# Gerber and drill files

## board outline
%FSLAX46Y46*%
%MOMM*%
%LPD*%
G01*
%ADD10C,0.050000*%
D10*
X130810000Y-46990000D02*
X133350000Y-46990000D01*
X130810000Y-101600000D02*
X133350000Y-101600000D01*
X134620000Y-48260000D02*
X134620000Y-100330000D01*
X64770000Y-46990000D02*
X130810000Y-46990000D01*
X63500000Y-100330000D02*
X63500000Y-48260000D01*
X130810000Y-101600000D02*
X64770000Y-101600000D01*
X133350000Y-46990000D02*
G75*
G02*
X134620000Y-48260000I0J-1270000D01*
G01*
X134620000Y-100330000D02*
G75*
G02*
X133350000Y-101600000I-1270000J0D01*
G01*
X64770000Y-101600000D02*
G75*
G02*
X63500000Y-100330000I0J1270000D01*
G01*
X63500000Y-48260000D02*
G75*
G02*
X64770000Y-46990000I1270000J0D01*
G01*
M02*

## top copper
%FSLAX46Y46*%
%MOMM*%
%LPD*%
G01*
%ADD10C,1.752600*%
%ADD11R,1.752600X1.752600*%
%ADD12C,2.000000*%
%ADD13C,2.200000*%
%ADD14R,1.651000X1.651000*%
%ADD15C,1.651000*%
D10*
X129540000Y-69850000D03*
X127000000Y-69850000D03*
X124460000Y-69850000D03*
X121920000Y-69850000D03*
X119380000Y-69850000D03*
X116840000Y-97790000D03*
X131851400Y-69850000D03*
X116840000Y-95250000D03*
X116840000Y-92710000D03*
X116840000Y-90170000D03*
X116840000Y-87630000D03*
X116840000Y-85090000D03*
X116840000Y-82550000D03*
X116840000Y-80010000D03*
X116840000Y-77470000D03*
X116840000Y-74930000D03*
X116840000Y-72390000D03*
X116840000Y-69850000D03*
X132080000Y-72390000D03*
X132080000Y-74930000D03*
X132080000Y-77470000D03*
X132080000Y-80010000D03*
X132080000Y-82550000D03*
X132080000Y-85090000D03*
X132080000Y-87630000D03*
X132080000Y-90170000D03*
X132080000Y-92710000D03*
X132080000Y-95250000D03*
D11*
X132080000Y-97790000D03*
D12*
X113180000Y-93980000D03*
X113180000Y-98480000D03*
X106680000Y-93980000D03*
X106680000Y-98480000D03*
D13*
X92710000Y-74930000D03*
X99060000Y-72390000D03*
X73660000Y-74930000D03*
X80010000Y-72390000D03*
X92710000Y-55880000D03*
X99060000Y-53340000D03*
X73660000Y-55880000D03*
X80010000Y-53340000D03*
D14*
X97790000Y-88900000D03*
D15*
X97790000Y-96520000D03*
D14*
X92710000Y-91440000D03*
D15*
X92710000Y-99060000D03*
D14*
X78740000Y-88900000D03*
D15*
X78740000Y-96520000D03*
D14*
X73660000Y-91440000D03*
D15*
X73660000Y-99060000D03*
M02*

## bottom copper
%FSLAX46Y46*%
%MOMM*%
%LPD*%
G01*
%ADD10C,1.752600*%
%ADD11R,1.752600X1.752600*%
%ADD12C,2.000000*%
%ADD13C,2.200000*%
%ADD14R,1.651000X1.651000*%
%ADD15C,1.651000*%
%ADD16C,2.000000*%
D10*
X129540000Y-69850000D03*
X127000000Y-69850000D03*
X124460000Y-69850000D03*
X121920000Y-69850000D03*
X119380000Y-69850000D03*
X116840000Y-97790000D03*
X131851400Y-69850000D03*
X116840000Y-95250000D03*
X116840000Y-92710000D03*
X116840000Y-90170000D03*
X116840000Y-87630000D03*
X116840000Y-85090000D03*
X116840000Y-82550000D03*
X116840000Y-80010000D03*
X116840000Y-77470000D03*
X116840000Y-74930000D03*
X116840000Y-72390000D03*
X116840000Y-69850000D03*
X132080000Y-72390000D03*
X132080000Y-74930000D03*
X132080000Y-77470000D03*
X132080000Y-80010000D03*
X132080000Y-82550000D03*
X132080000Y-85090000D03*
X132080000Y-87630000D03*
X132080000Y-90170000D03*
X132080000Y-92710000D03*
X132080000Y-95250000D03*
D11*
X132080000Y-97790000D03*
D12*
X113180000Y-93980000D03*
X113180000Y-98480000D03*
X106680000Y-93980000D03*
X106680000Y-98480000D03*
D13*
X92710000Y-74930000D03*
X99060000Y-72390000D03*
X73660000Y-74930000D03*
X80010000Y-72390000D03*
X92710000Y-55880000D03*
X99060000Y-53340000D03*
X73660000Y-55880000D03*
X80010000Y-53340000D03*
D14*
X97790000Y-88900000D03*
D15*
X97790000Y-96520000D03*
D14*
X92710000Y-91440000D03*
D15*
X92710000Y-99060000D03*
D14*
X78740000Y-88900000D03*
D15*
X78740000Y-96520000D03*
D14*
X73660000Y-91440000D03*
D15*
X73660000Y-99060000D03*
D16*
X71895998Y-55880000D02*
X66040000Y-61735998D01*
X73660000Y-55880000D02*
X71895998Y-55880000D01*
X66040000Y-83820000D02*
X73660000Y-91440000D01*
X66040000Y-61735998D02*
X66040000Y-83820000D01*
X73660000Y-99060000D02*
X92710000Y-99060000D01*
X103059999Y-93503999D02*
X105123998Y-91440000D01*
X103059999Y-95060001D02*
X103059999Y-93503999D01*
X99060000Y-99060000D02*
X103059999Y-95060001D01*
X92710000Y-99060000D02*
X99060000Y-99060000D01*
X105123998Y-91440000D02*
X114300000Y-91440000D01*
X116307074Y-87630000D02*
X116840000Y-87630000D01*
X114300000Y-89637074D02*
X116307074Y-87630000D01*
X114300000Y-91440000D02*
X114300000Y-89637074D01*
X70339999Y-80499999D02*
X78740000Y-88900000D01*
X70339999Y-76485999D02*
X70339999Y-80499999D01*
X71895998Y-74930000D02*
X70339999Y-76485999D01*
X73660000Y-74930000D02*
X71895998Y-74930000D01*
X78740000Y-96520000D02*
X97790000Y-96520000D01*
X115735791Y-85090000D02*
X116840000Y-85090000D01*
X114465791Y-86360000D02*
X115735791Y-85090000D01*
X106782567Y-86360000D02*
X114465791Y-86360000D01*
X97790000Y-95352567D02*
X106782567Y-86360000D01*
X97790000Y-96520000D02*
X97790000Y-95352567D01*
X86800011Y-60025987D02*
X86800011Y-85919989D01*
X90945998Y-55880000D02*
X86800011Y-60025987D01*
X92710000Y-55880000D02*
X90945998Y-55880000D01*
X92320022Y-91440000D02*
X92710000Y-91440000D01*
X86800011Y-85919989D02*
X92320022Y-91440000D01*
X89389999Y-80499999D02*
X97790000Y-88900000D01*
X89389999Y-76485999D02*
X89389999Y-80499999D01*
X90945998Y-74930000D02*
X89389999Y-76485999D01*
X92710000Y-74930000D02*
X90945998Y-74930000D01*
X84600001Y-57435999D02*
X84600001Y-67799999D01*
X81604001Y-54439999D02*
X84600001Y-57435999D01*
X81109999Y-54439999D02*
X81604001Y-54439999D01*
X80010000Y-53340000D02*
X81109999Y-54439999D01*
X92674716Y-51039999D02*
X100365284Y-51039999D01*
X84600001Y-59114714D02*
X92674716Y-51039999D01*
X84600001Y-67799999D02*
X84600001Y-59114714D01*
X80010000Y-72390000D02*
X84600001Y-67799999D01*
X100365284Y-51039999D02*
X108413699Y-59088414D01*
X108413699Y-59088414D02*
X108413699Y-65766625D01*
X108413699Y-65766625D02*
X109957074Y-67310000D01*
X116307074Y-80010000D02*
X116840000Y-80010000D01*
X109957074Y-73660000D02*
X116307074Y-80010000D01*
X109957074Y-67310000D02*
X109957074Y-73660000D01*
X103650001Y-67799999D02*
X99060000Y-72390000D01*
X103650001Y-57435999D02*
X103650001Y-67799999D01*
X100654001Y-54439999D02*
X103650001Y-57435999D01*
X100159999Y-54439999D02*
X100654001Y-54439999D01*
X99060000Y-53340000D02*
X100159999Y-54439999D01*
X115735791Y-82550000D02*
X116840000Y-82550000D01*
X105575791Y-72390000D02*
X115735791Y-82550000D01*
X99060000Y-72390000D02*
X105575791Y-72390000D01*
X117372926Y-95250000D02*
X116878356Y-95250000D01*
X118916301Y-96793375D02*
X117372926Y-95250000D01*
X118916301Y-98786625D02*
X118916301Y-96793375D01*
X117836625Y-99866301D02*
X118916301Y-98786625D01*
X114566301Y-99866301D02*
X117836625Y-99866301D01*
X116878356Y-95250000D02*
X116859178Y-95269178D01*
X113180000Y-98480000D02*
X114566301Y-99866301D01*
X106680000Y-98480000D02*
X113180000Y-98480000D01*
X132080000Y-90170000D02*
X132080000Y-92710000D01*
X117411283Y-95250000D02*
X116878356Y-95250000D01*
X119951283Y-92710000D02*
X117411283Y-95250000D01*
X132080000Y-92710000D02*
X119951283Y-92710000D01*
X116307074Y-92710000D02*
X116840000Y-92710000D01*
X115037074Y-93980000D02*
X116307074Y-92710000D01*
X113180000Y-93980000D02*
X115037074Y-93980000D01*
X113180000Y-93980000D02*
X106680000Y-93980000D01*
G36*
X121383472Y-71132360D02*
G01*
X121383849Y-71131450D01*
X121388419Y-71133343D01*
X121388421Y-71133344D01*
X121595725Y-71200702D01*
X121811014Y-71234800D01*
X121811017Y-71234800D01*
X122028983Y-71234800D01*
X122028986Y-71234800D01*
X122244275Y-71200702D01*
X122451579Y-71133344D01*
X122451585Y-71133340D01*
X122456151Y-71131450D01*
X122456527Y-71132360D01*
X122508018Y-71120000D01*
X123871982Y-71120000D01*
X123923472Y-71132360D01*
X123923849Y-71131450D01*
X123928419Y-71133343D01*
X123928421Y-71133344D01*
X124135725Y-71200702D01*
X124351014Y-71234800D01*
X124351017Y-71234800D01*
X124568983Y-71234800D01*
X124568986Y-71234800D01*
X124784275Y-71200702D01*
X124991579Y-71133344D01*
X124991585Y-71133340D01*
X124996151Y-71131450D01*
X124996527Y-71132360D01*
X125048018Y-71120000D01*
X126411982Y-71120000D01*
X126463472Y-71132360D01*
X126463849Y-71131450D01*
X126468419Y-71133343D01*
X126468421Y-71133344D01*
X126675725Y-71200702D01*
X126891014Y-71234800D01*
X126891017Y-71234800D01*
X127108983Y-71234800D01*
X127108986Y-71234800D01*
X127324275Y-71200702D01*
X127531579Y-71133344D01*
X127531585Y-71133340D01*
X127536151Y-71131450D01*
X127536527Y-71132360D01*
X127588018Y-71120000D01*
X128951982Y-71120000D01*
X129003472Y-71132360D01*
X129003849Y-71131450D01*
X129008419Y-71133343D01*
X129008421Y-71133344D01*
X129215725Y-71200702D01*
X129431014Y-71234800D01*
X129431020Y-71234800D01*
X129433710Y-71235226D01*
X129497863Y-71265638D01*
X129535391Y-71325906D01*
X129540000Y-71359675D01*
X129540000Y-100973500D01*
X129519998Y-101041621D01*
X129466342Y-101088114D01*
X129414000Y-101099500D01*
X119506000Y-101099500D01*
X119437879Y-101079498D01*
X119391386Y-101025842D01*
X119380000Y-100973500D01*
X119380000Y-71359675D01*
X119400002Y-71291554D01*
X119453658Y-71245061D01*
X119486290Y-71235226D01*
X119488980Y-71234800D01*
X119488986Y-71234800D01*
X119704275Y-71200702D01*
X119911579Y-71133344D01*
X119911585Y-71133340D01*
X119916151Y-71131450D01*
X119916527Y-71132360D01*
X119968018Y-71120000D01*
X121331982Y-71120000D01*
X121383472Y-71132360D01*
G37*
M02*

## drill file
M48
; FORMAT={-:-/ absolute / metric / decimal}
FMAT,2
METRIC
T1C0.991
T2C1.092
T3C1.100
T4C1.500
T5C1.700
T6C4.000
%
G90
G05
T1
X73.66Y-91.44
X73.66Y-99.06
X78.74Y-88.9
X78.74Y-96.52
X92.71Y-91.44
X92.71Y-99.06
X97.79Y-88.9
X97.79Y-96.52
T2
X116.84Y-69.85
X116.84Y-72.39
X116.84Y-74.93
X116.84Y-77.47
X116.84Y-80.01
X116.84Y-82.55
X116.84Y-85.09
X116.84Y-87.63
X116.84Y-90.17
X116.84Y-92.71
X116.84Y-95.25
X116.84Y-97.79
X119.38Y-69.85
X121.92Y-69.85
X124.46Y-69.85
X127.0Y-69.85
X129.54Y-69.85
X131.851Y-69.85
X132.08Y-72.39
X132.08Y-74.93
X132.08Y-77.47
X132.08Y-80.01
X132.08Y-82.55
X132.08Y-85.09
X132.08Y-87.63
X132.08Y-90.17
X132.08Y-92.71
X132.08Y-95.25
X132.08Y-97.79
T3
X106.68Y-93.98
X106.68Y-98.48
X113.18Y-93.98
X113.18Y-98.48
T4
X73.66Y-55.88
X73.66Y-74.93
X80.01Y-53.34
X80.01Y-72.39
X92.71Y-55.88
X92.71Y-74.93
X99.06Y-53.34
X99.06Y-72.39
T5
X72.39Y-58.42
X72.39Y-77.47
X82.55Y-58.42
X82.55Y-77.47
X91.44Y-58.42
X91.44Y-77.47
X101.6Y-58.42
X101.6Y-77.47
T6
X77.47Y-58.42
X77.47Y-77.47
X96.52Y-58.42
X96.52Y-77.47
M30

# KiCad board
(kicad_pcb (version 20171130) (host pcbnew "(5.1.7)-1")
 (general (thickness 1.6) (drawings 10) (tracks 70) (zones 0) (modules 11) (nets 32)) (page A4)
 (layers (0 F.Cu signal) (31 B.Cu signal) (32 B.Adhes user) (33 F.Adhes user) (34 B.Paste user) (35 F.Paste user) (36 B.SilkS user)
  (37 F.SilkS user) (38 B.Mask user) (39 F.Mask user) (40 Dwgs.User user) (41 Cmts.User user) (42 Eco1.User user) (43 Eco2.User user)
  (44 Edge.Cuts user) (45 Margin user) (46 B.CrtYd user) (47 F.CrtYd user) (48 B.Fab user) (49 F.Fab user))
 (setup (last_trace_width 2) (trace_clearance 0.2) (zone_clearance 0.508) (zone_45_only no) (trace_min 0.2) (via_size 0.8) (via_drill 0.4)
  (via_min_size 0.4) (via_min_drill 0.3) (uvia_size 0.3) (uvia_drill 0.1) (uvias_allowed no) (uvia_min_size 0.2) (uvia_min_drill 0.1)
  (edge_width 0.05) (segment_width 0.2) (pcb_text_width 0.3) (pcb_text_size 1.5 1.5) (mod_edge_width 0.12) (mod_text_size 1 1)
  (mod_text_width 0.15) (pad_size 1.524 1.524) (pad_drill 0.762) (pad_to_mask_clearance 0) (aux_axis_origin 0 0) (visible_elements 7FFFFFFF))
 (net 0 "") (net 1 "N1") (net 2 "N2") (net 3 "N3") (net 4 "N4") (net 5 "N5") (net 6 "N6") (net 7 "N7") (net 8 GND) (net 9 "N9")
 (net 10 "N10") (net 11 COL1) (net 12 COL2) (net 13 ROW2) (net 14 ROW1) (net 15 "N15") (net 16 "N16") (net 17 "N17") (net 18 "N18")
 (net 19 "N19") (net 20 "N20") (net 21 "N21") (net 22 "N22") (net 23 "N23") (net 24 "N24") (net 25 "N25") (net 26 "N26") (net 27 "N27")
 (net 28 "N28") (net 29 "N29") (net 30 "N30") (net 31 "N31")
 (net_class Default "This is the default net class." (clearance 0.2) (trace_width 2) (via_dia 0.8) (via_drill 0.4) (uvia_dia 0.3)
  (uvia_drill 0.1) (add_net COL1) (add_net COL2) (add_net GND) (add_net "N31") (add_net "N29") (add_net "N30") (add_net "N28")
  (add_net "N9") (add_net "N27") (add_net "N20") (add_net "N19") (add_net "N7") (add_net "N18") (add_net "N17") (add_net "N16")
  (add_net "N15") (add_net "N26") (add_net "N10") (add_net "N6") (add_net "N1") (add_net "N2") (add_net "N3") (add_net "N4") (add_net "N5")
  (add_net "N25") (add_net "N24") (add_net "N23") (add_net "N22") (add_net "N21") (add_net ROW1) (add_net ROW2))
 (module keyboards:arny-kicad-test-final (layer F.Cu) (at 124.46 57.15)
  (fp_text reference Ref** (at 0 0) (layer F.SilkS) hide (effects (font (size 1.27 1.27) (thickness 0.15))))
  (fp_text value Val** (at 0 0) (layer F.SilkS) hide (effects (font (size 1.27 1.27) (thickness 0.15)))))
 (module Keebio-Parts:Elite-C (layer F.Cu) (at 124.46 83.82 90)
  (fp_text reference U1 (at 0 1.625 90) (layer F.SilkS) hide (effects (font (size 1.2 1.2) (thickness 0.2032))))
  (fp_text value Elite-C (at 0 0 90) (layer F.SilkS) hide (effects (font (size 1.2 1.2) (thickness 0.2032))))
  (pad 25 thru_hole circle (at 13.97 5.08 90) (size 1.7526 1.7526) (drill 1.0922) (layers *.Cu *.SilkS *.Mask) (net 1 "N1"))
  (pad 26 thru_hole circle (at 13.97 2.54 90) (size 1.7526 1.7526) (drill 1.0922) (layers *.Cu *.SilkS *.Mask) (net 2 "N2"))
  (pad 27 thru_hole circle (at 13.97 0 90) (size 1.7526 1.7526) (drill 1.0922) (layers *.Cu *.SilkS *.Mask) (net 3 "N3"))
  (pad 28 thru_hole circle (at 13.97 -2.54 90) (size 1.7526 1.7526) (drill 1.0922) (layers *.Cu *.SilkS *.Mask) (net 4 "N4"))
  (pad 29 thru_hole circle (at 13.97 -5.08 90) (size 1.7526 1.7526) (drill 1.0922) (layers *.Cu *.SilkS *.Mask) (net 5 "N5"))
  (pad 24 thru_hole circle (at -13.97 -7.62 90) (size 1.7526 1.7526) (drill 1.0922) (layers *.Cu *.SilkS *.Mask) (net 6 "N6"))
  (pad 12 thru_hole circle (at 13.97 7.3914 90) (size 1.7526 1.7526) (drill 1.0922) (layers *.Cu *.SilkS *.Mask) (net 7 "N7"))
  (pad 23 thru_hole circle (at -11.43 -7.62 90) (size 1.7526 1.7526) (drill 1.0922) (layers *.Cu *.SilkS *.Mask) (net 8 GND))
  (pad 22 thru_hole circle (at -8.89 -7.62 90) (size 1.7526 1.7526) (drill 1.0922) (layers *.Cu *.SilkS *.Mask) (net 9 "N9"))
  (pad 21 thru_hole circle (at -6.35 -7.62 90) (size 1.7526 1.7526) (drill 1.0922) (layers *.Cu *.SilkS *.Mask) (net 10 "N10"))
  (pad 20 thru_hole circle (at -3.81 -7.62 90) (size 1.7526 1.7526) (drill 1.0922) (layers *.Cu *.SilkS *.Mask) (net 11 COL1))
  (pad 19 thru_hole circle (at -1.27 -7.62 90) (size 1.7526 1.7526) (drill 1.0922) (layers *.Cu *.SilkS *.Mask) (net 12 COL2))
  (pad 18 thru_hole circle (at 1.27 -7.62 90) (size 1.7526 1.7526) (drill 1.0922) (layers *.Cu *.SilkS *.Mask) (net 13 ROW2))
  (pad 17 thru_hole circle (at 3.81 -7.62 90) (size 1.7526 1.7526) (drill 1.0922) (layers *.Cu *.SilkS *.Mask) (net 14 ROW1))
  (pad 16 thru_hole circle (at 6.35 -7.62 90) (size 1.7526 1.7526) (drill 1.0922) (layers *.Cu *.SilkS *.Mask) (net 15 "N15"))
  (pad 15 thru_hole circle (at 8.89 -7.62 90) (size 1.7526 1.7526) (drill 1.0922) (layers *.Cu *.SilkS *.Mask) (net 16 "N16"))
  (pad 14 thru_hole circle (at 11.43 -7.62 90) (size 1.7526 1.7526) (drill 1.0922) (layers *.Cu *.SilkS *.Mask) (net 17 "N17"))
  (pad 13 thru_hole circle (at 13.97 -7.62 90) (size 1.7526 1.7526) (drill 1.0922) (layers *.Cu *.SilkS *.Mask) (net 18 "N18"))
  (pad 11 thru_hole circle (at 11.43 7.62 90) (size 1.7526 1.7526) (drill 1.0922) (layers *.Cu *.SilkS *.Mask) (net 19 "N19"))
  (pad 10 thru_hole circle (at 8.89 7.62 90) (size 1.7526 1.7526) (drill 1.0922) (layers *.Cu *.SilkS *.Mask) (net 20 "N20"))
  (pad 9 thru_hole circle (at 6.35 7.62 90) (size 1.7526 1.7526) (drill 1.0922) (layers *.Cu *.SilkS *.Mask) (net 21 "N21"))
  (pad 8 thru_hole circle (at 3.81 7.62 90) (size 1.7526 1.7526) (drill 1.0922) (layers *.Cu *.SilkS *.Mask) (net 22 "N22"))
  (pad 7 thru_hole circle (at 1.27 7.62 90) (size 1.7526 1.7526) (drill 1.0922) (layers *.Cu *.SilkS *.Mask) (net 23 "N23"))
  (pad 6 thru_hole circle (at -1.27 7.62 90) (size 1.7526 1.7526) (drill 1.0922) (layers *.Cu *.SilkS *.Mask) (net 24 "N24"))
  (pad 5 thru_hole circle (at -3.81 7.62 90) (size 1.7526 1.7526) (drill 1.0922) (layers *.Cu *.SilkS *.Mask) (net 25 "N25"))
  (pad 4 thru_hole circle (at -6.35 7.62 90) (size 1.7526 1.7526) (drill 1.0922) (layers *.Cu *.SilkS *.Mask) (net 8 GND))
  (pad 3 thru_hole circle (at -8.89 7.62 90) (size 1.7526 1.7526) (drill 1.0922) (layers *.Cu *.SilkS *.Mask) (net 8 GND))
  (pad 2 thru_hole circle (at -11.43 7.62 90) (size 1.7526 1.7526) (drill 1.0922) (layers *.Cu *.SilkS *.Mask) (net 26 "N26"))
  (pad 1 thru_hole rect (at -13.97 7.62 90) (size 1.7526 1.7526) (drill 1.0922) (layers *.Cu *.SilkS *.Mask) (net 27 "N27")))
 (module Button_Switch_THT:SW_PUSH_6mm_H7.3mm (layer F.Cu) (at 106.68 93.98)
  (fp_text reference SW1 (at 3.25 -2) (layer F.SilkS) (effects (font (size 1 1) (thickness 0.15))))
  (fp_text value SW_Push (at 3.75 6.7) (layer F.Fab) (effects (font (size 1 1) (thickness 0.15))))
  (pad 1 thru_hole circle (at 6.5 0 90) (size 2 2) (drill 1.1) (layers *.Cu *.Mask) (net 9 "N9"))
  (pad 2 thru_hole circle (at 6.5 4.5 90) (size 2 2) (drill 1.1) (layers *.Cu *.Mask) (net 8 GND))
  (pad 1 thru_hole circle (at 0 0 90) (size 2 2) (drill 1.1) (layers *.Cu *.Mask) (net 9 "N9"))
  (pad 2 thru_hole circle (at 0 4.5 90) (size 2 2) (drill 1.1) (layers *.Cu *.Mask) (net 8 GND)))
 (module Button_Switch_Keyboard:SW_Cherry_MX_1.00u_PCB (layer F.Cu) (at 99.06 72.39)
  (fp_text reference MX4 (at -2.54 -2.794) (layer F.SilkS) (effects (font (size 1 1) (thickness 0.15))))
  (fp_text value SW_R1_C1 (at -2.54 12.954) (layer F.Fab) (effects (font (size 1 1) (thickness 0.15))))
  (pad "" np_thru_hole circle (at 2.54 5.08) (size 1.7 1.7) (drill 1.7) (layers *.Cu *.Mask))
  (pad "" np_thru_hole circle (at -7.62 5.08) (size 1.7 1.7) (drill 1.7) (layers *.Cu *.Mask))
  (pad "" np_thru_hole circle (at -2.54 5.08) (size 4 4) (drill 4) (layers *.Cu *.Mask))
  (pad 2 thru_hole circle (at -6.35 2.54) (size 2.2 2.2) (drill 1.5) (layers *.Cu *.Mask) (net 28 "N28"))
  (pad 1 thru_hole circle (at 0 0) (size 2.2 2.2) (drill 1.5) (layers *.Cu *.Mask) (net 13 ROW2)))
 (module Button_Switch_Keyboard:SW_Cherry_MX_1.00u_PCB (layer F.Cu) (at 80.01 72.39)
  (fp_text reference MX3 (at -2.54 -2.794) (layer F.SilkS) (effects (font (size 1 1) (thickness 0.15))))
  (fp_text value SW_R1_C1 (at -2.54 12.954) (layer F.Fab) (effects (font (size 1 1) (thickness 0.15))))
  (pad "" np_thru_hole circle (at 2.54 5.08) (size 1.7 1.7) (drill 1.7) (layers *.Cu *.Mask))
  (pad "" np_thru_hole circle (at -7.62 5.08) (size 1.7 1.7) (drill 1.7) (layers *.Cu *.Mask))
  (pad "" np_thru_hole circle (at -2.54 5.08) (size 4 4) (drill 4) (layers *.Cu *.Mask))
  (pad 2 thru_hole circle (at -6.35 2.54) (size 2.2 2.2) (drill 1.5) (layers *.Cu *.Mask) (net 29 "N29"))
  (pad 1 thru_hole circle (at 0 0) (size 2.2 2.2) (drill 1.5) (layers *.Cu *.Mask) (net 14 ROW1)))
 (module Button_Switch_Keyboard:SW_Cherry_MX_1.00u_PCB (layer F.Cu) (at 99.06 53.34)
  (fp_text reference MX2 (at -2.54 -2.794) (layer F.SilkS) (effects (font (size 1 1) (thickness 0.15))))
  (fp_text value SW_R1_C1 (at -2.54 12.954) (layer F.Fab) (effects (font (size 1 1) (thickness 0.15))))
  (pad "" np_thru_hole circle (at 2.54 5.08) (size 1.7 1.7) (drill 1.7) (layers *.Cu *.Mask))
  (pad "" np_thru_hole circle (at -7.62 5.08) (size 1.7 1.7) (drill 1.7) (layers *.Cu *.Mask))
  (pad "" np_thru_hole circle (at -2.54 5.08) (size 4 4) (drill 4) (layers *.Cu *.Mask))
  (pad 2 thru_hole circle (at -6.35 2.54) (size 2.2 2.2) (drill 1.5) (layers *.Cu *.Mask) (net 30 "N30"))
  (pad 1 thru_hole circle (at 0 0) (size 2.2 2.2) (drill 1.5) (layers *.Cu *.Mask) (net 13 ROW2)))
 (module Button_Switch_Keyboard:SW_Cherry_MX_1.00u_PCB (layer F.Cu) (at 80.01 53.34)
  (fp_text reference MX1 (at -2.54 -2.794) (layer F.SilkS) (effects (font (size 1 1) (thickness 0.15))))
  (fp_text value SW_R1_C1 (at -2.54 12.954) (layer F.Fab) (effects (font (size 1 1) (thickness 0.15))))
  (pad "" np_thru_hole circle (at 2.54 5.08) (size 1.7 1.7) (drill 1.7) (layers *.Cu *.Mask))
  (pad "" np_thru_hole circle (at -7.62 5.08) (size 1.7 1.7) (drill 1.7) (layers *.Cu *.Mask))
  (pad "" np_thru_hole circle (at -2.54 5.08) (size 4 4) (drill 4) (layers *.Cu *.Mask))
  (pad 2 thru_hole circle (at -6.35 2.54) (size 2.2 2.2) (drill 1.5) (layers *.Cu *.Mask) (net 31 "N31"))
  (pad 1 thru_hole circle (at 0 0) (size 2.2 2.2) (drill 1.5) (layers *.Cu *.Mask) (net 14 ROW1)))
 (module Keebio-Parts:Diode (layer F.Cu) (at 97.79 92.71 90)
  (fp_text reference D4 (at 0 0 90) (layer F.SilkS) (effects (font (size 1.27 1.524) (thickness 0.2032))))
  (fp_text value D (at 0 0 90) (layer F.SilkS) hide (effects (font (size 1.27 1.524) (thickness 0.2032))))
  (pad 2 thru_hole rect (at 3.81 0 90) (size 1.651 1.651) (drill 0.9906) (layers *.Cu *.SilkS *.Mask) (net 28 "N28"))
  (pad 1 thru_hole circle (at -3.81 0 90) (size 1.651 1.651) (drill 0.9906) (layers *.Cu *.SilkS *.Mask) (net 12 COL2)))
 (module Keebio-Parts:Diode (layer F.Cu) (at 92.71 95.25 90)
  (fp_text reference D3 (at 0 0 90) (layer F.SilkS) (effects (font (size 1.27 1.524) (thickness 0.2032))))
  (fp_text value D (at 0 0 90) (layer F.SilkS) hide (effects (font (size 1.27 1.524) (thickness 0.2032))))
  (pad 2 thru_hole rect (at 3.81 0 90) (size 1.651 1.651) (drill 0.9906) (layers *.Cu *.SilkS *.Mask) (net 30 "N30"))
  (pad 1 thru_hole circle (at -3.81 0 90) (size 1.651 1.651) (drill 0.9906) (layers *.Cu *.SilkS *.Mask) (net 11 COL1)))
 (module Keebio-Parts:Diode (layer F.Cu) (at 78.74 92.71 90)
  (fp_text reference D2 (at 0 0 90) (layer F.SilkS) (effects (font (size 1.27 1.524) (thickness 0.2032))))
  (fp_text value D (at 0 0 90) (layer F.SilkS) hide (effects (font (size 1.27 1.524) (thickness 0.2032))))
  (pad 2 thru_hole rect (at 3.81 0 90) (size 1.651 1.651) (drill 0.9906) (layers *.Cu *.SilkS *.Mask) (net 29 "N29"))
  (pad 1 thru_hole circle (at -3.81 0 90) (size 1.651 1.651) (drill 0.9906) (layers *.Cu *.SilkS *.Mask) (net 12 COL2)))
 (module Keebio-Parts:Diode (layer F.Cu) (at 73.66 95.25 90)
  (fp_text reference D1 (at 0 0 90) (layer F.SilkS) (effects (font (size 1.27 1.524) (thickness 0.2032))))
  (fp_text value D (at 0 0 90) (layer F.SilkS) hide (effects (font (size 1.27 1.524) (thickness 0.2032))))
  (pad 2 thru_hole rect (at 3.81 0 90) (size 1.651 1.651) (drill 0.9906) (layers *.Cu *.SilkS *.Mask) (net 31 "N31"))
  (pad 1 thru_hole circle (at -3.81 0 90) (size 1.651 1.651) (drill 0.9906) (layers *.Cu *.SilkS *.Mask) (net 11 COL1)))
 (gr_line (start 130.81 46.99) (end 133.35 46.99) (layer Edge.Cuts) (width 0.05))
 (gr_line (start 130.81 101.6) (end 133.35 101.6) (layer Edge.Cuts) (width 0.05))
 (gr_line (start 134.62 48.26) (end 134.62 100.33) (layer Edge.Cuts) (width 0.05))
 (gr_line (start 64.77 46.99) (end 130.81 46.99) (layer Edge.Cuts) (width 0.05))
 (gr_line (start 63.5 100.33) (end 63.5 48.26) (layer Edge.Cuts) (width 0.05))
 (gr_line (start 130.81 101.6) (end 64.77 101.6) (layer Edge.Cuts) (width 0.05))
 (gr_arc (start 133.35 48.26) (end 134.62 48.26) (angle -90) (layer Edge.Cuts) (width 0.05))
 (gr_arc (start 133.35 100.33) (end 133.35 101.6) (angle -90) (layer Edge.Cuts) (width 0.05))
 (gr_arc (start 64.77 100.33) (end 63.5 100.33) (angle -90) (layer Edge.Cuts) (width 0.05))
 (gr_arc (start 64.77 48.26) (end 64.77 46.99) (angle -90) (layer Edge.Cuts) (width 0.05))
 (segment (start 71.895998 55.88) (end 66.04 61.735998) (width 2) (layer B.Cu) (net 31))
 (segment (start 73.66 55.88) (end 71.895998 55.88) (width 2) (layer B.Cu) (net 31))
 (segment (start 66.04 83.82) (end 73.66 91.44) (width 2) (layer B.Cu) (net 31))
 (segment (start 66.04 61.735998) (end 66.04 83.82) (width 2) (layer B.Cu) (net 31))
 (segment (start 73.66 99.06) (end 92.71 99.06) (width 2) (layer B.Cu) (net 11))
 (segment (start 103.059999 93.503999) (end 105.123998 91.44) (width 2) (layer B.Cu) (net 11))
 (segment (start 103.059999 95.060001) (end 103.059999 93.503999) (width 2) (layer B.Cu) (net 11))
 (segment (start 99.06 99.06) (end 103.059999 95.060001) (width 2) (layer B.Cu) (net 11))
 (segment (start 92.71 99.06) (end 99.06 99.06) (width 2) (layer B.Cu) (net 11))
 (segment (start 105.123998 91.44) (end 114.3 91.44) (width 2) (layer B.Cu) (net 11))
 (segment (start 116.307074 87.63) (end 116.84 87.63) (width 2) (layer B.Cu) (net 11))
 (segment (start 114.3 89.637074) (end 116.307074 87.63) (width 2) (layer B.Cu) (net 11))
 (segment (start 114.3 91.44) (end 114.3 89.637074) (width 2) (layer B.Cu) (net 11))
 (segment (start 70.339999 80.499999) (end 78.74 88.9) (width 2) (layer B.Cu) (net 29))
 (segment (start 70.339999 76.485999) (end 70.339999 80.499999) (width 2) (layer B.Cu) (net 29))
 (segment (start 71.895998 74.93) (end 70.339999 76.485999) (width 2) (layer B.Cu) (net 29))
 (segment (start 73.66 74.93) (end 71.895998 74.93) (width 2) (layer B.Cu) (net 29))
 (segment (start 78.74 96.52) (end 97.79 96.52) (width 2) (layer B.Cu) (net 12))
 (segment (start 115.735791 85.09) (end 116.84 85.09) (width 2) (layer B.Cu) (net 12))
 (segment (start 114.465791 86.36) (end 115.735791 85.09) (width 2) (layer B.Cu) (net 12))
 (segment (start 106.782567 86.36) (end 114.465791 86.36) (width 2) (layer B.Cu) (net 12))
 (segment (start 97.79 95.352567) (end 106.782567 86.36) (width 2) (layer B.Cu) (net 12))
 (segment (start 97.79 96.52) (end 97.79 95.352567) (width 2) (layer B.Cu) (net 12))
 (segment (start 86.800011 60.025987) (end 86.800011 85.919989) (width 2) (layer B.Cu) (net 30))
 (segment (start 90.945998 55.88) (end 86.800011 60.025987) (width 2) (layer B.Cu) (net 30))
 (segment (start 92.71 55.88) (end 90.945998 55.88) (width 2) (layer B.Cu) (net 30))
 (segment (start 92.320022 91.44) (end 92.71 91.44) (width 2) (layer B.Cu) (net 30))
 (segment (start 86.800011 85.919989) (end 92.320022 91.44) (width 2) (layer B.Cu) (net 30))
 (segment (start 89.389999 80.499999) (end 97.79 88.9) (width 2) (layer B.Cu) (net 28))
 (segment (start 89.389999 76.485999) (end 89.389999 80.499999) (width 2) (layer B.Cu) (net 28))
 (segment (start 90.945998 74.93) (end 89.389999 76.485999) (width 2) (layer B.Cu) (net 28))
 (segment (start 92.71 74.93) (end 90.945998 74.93) (width 2) (layer B.Cu) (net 28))
 (segment (start 84.600001 57.435999) (end 84.600001 67.799999) (width 2) (layer B.Cu) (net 14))
 (segment (start 81.604001 54.439999) (end 84.600001 57.435999) (width 2) (layer B.Cu) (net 14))
 (segment (start 81.109999 54.439999) (end 81.604001 54.439999) (width 2) (layer B.Cu) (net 14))
 (segment (start 80.01 53.34) (end 81.109999 54.439999) (width 2) (layer B.Cu) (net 14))
 (segment (start 92.674716 51.039999) (end 100.365284 51.039999) (width 2) (layer B.Cu) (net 14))
 (segment (start 84.600001 59.114714) (end 92.674716 51.039999) (width 2) (layer B.Cu) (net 14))
 (segment (start 84.600001 67.799999) (end 84.600001 59.114714) (width 2) (layer B.Cu) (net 14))
 (segment (start 80.01 72.39) (end 84.600001 67.799999) (width 2) (layer B.Cu) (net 14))
 (segment (start 100.365284 51.039999) (end 108.413699 59.088414) (width 2) (layer B.Cu) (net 14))
 (segment (start 108.413699 59.088414) (end 108.413699 65.766625) (width 2) (layer B.Cu) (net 14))
 (segment (start 108.413699 65.766625) (end 109.957074 67.31) (width 2) (layer B.Cu) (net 14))
 (segment (start 116.307074 80.01) (end 116.84 80.01) (width 2) (layer B.Cu) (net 14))
 (segment (start 109.957074 73.66) (end 116.307074 80.01) (width 2) (layer B.Cu) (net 14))
 (segment (start 109.957074 67.31) (end 109.957074 73.66) (width 2) (layer B.Cu) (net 14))
 (segment (start 103.650001 67.799999) (end 99.06 72.39) (width 2) (layer B.Cu) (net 13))
 (segment (start 103.650001 57.435999) (end 103.650001 67.799999) (width 2) (layer B.Cu) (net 13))
 (segment (start 100.654001 54.439999) (end 103.650001 57.435999) (width 2) (layer B.Cu) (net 13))
 (segment (start 100.159999 54.439999) (end 100.654001 54.439999) (width 2) (layer B.Cu) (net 13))
 (segment (start 99.06 53.34) (end 100.159999 54.439999) (width 2) (layer B.Cu) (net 13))
 (segment (start 115.735791 82.55) (end 116.84 82.55) (width 2) (layer B.Cu) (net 13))
 (segment (start 105.575791 72.39) (end 115.735791 82.55) (width 2) (layer B.Cu) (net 13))
 (segment (start 99.06 72.39) (end 105.575791 72.39) (width 2) (layer B.Cu) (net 13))
 (segment (start 117.372926 95.25) (end 116.878356 95.25) (width 2) (layer B.Cu) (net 8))
 (segment (start 118.916301 96.793375) (end 117.372926 95.25) (width 2) (layer B.Cu) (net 8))
 (segment (start 118.916301 98.786625) (end 118.916301 96.793375) (width 2) (layer B.Cu) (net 8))
 (segment (start 117.836625 99.866301) (end 118.916301 98.786625) (width 2) (layer B.Cu) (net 8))
 (segment (start 114.566301 99.866301) (end 117.836625 99.866301) (width 2) (layer B.Cu) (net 8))
 (segment (start 116.878356 95.25) (end 116.859178 95.269178) (width 2) (layer B.Cu) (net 8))
 (segment (start 113.18 98.48) (end 114.566301 99.866301) (width 2) (layer B.Cu) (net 8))
 (segment (start 106.68 98.48) (end 113.18 98.48) (width 2) (layer B.Cu) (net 8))
 (segment (start 132.08 90.17) (end 132.08 92.71) (width 2) (layer B.Cu) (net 8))
 (segment (start 117.411283 95.25) (end 116.878356 95.25) (width 2) (layer B.Cu) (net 8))
 (segment (start 119.951283 92.71) (end 117.411283 95.25) (width 2) (layer B.Cu) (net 8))
 (segment (start 132.08 92.71) (end 119.951283 92.71) (width 2) (layer B.Cu) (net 8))
 (segment (start 116.307074 92.71) (end 116.84 92.71) (width 2) (layer B.Cu) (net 9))
 (segment (start 115.037074 93.98) (end 116.307074 92.71) (width 2) (layer B.Cu) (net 9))
 (segment (start 113.18 93.98) (end 115.037074 93.98) (width 2) (layer B.Cu) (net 9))
 (segment (start 113.18 93.98) (end 106.68 93.98) (width 2) (layer B.Cu) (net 9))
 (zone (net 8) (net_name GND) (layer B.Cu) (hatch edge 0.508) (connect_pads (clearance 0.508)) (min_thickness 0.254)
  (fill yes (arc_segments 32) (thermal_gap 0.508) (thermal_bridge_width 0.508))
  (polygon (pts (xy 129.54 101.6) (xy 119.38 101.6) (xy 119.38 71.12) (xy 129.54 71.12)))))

